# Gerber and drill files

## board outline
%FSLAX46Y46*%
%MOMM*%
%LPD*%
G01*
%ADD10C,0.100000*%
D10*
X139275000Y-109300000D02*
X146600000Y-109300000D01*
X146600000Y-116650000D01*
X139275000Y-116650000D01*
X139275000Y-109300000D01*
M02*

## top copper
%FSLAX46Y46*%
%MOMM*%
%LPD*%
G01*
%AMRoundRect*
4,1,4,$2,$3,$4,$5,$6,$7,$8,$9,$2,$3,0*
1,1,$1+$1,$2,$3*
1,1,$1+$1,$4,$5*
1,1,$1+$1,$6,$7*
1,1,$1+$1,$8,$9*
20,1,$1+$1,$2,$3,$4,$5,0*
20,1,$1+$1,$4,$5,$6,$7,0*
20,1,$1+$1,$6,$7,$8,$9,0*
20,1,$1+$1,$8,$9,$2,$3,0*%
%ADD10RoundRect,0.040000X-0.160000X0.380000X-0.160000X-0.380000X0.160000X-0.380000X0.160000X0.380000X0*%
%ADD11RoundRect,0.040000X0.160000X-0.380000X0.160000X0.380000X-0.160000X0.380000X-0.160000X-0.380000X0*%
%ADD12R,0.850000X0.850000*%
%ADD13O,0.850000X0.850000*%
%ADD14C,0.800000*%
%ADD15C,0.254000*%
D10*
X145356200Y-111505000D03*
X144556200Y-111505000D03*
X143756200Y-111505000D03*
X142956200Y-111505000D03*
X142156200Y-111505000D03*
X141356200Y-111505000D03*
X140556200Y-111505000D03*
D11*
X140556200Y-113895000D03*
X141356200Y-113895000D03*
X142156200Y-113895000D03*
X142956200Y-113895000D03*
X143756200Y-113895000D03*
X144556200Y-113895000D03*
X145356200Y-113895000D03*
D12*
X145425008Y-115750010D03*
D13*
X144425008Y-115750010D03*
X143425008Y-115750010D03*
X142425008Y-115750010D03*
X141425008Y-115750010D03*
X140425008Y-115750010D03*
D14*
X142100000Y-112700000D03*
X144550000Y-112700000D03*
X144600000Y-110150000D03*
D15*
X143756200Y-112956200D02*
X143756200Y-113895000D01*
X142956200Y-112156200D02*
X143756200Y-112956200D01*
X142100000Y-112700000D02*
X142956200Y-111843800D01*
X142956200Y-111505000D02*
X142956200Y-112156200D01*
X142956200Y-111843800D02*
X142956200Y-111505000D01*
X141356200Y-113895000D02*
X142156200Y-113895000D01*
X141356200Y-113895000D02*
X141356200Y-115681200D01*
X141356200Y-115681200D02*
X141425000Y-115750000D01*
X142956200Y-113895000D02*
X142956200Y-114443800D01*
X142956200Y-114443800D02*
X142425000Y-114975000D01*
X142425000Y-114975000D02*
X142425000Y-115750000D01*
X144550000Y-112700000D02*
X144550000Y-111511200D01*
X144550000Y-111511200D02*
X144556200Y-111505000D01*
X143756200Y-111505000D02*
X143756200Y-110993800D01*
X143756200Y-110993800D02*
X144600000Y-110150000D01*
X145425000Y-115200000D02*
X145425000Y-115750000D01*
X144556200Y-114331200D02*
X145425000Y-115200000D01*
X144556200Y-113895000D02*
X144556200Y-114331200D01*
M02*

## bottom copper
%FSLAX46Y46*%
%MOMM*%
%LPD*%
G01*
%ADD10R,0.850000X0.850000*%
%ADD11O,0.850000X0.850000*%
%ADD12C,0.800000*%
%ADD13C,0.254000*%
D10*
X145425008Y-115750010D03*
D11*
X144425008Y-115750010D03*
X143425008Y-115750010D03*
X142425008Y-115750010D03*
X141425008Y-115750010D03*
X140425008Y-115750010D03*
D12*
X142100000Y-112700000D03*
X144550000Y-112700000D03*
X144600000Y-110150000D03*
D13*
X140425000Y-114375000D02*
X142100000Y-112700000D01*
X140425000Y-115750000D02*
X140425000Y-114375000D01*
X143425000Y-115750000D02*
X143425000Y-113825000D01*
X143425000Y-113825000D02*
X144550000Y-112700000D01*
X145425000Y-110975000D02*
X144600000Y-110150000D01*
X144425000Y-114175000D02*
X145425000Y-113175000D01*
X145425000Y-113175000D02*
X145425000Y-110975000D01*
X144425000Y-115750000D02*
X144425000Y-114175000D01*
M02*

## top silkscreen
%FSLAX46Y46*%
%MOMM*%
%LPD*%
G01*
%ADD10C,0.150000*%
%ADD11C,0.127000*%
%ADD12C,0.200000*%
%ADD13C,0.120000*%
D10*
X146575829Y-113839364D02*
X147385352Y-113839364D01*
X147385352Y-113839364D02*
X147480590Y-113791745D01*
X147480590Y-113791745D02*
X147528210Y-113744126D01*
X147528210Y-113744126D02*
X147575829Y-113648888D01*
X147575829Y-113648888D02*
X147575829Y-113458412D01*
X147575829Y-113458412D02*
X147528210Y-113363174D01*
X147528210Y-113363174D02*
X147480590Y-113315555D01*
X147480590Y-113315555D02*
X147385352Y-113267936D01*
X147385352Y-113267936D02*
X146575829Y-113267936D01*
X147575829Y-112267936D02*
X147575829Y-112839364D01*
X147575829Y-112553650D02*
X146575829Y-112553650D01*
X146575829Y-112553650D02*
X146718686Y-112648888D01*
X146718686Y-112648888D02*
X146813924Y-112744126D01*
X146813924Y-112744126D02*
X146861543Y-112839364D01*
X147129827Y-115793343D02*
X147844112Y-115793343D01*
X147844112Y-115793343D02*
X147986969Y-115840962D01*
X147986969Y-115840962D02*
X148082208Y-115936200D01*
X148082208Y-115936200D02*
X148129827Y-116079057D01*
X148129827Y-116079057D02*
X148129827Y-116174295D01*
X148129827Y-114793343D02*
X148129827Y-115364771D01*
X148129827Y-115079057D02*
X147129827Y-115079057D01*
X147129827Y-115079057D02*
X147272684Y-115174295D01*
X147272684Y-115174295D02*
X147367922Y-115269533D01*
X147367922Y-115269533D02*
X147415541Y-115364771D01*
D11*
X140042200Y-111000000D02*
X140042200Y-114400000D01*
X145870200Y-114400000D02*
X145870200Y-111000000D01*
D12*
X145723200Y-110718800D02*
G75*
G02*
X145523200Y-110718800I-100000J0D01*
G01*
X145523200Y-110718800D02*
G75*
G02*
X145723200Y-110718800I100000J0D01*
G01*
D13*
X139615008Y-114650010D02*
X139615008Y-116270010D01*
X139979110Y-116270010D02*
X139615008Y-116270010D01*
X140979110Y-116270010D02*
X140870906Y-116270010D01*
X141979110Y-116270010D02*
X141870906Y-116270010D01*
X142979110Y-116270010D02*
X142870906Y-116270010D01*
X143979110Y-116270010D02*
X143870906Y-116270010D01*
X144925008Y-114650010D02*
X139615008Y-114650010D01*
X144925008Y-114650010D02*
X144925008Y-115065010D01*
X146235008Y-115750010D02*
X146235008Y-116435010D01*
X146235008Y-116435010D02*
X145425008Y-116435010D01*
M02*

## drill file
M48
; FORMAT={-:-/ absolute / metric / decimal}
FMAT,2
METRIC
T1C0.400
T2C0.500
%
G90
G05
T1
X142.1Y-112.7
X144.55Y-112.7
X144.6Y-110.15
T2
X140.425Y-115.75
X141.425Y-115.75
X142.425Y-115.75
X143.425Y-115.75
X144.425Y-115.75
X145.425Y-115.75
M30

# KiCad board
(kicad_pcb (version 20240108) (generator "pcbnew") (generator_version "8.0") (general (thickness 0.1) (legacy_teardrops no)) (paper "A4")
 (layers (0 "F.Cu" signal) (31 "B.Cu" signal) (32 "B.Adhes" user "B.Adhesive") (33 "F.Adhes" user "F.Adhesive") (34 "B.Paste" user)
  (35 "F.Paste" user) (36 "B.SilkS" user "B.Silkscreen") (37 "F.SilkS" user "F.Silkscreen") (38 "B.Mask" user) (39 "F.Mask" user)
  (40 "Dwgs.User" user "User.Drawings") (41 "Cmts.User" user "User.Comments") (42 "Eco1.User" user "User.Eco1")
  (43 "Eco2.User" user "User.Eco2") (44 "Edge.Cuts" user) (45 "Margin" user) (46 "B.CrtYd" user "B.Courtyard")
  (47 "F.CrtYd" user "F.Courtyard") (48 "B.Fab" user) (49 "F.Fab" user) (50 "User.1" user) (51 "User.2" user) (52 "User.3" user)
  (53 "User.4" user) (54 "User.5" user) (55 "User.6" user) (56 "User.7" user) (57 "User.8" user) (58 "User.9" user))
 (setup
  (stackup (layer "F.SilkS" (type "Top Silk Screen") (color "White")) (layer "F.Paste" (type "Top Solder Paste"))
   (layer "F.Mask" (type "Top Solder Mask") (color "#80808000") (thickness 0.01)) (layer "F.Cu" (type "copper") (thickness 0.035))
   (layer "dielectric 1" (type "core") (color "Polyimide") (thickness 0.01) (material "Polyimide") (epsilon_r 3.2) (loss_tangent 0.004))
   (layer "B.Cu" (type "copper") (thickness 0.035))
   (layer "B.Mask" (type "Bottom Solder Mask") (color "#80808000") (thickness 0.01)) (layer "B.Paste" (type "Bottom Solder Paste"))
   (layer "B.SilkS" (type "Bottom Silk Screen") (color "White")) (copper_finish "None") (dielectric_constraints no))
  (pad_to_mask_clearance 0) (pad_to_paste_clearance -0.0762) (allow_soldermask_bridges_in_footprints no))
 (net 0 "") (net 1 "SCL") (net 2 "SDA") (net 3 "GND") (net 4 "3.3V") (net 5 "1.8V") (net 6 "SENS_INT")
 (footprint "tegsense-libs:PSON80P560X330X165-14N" (layer "F.Cu") (at 142.9562 112.7 -90)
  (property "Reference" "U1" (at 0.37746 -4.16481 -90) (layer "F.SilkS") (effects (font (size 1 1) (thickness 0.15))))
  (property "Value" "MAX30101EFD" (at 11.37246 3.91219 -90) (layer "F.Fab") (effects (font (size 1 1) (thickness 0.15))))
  (fp_line (start -1.7 2.914) (end 1.7 2.914) (stroke (width 0.127) (type solid)) (layer "F.SilkS"))
  (fp_line (start 1.7 -2.914) (end -1.7 -2.914) (stroke (width 0.127) (type solid)) (layer "F.SilkS"))
  (fp_circle (center -1.9812 -2.667) (end -1.8812 -2.667) (stroke (width 0.2) (type solid)) (fill none) (layer "F.SilkS"))
  (pad "1" smd roundrect (at -1.195 -2.4 270) (size 0.84 0.4) (layers "F.Cu" "F.Paste" "F.Mask") (roundrect_rratio 0.1))
  (pad "2" smd roundrect (at -1.195 -1.6 270) (size 0.84 0.4) (layers "F.Cu" "F.Paste" "F.Mask") (roundrect_rratio 0.1) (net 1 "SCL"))
  (pad "3" smd roundrect (at -1.195 -0.8 270) (size 0.84 0.4) (layers "F.Cu" "F.Paste" "F.Mask") (roundrect_rratio 0.1) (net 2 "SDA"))
  (pad "4" smd roundrect (at -1.195 0 270) (size 0.84 0.4) (layers "F.Cu" "F.Paste" "F.Mask") (roundrect_rratio 0.1) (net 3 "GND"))
  (pad "5" smd roundrect (at -1.195 0.8 270) (size 0.84 0.4) (layers "F.Cu" "F.Paste" "F.Mask") (roundrect_rratio 0.1))
  (pad "6" smd roundrect (at -1.195 1.6 270) (size 0.84 0.4) (layers "F.Cu" "F.Paste" "F.Mask") (roundrect_rratio 0.1))
  (pad "7" smd roundrect (at -1.195 2.4 270) (size 0.84 0.4) (layers "F.Cu" "F.Paste" "F.Mask") (roundrect_rratio 0.1))
  (pad "8" smd roundrect (at 1.195 2.4 90) (size 0.84 0.4) (layers "F.Cu" "F.Paste" "F.Mask") (roundrect_rratio 0.1))
  (pad "9" smd roundrect (at 1.195 1.6 90) (size 0.84 0.4) (layers "F.Cu" "F.Paste" "F.Mask") (roundrect_rratio 0.1) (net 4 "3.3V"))
  (pad "10" smd roundrect (at 1.195 0.8 90) (size 0.84 0.4) (layers "F.Cu" "F.Paste" "F.Mask") (roundrect_rratio 0.1) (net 4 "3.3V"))
  (pad "11" smd roundrect (at 1.195 0 90) (size 0.84 0.4) (layers "F.Cu" "F.Paste" "F.Mask") (roundrect_rratio 0.1) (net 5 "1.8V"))
  (pad "12" smd roundrect (at 1.195 -0.8 90) (size 0.84 0.4) (layers "F.Cu" "F.Paste" "F.Mask") (roundrect_rratio 0.1) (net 3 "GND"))
  (pad "13" smd roundrect (at 1.195 -1.6 90) (size 0.84 0.4) (layers "F.Cu" "F.Paste" "F.Mask") (roundrect_rratio 0.1) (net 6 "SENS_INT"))
  (pad "14" smd roundrect (at 1.195 -2.4 90) (size 0.84 0.4) (layers "F.Cu" "F.Paste" "F.Mask") (roundrect_rratio 0.1)))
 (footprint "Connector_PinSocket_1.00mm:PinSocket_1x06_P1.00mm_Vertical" (layer "F.Cu") (at 145.425008 115.75001 -90)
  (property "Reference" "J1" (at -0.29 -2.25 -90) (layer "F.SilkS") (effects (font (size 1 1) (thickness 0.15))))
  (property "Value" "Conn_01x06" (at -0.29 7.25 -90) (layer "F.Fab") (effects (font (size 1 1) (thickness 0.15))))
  (fp_line (start -1.1 5.81) (end 0.52 5.81) (stroke (width 0.12) (type solid)) (layer "F.SilkS"))
  (fp_line (start 0.52 5.445898) (end 0.52 5.81) (stroke (width 0.12) (type solid)) (layer "F.SilkS"))
  (fp_line (start 0.52 4.445898) (end 0.52 4.554102) (stroke (width 0.12) (type solid)) (layer "F.SilkS"))
  (fp_line (start 0.52 3.445898) (end 0.52 3.554102) (stroke (width 0.12) (type solid)) (layer "F.SilkS"))
  (fp_line (start 0.52 2.445898) (end 0.52 2.554102) (stroke (width 0.12) (type solid)) (layer "F.SilkS"))
  (fp_line (start 0.52 1.445898) (end 0.52 1.554102) (stroke (width 0.12) (type solid)) (layer "F.SilkS"))
  (fp_line (start -1.1 0.5) (end -1.1 5.81) (stroke (width 0.12) (type solid)) (layer "F.SilkS"))
  (fp_line (start -1.1 0.5) (end -0.685 0.5) (stroke (width 0.12) (type solid)) (layer "F.SilkS"))
  (fp_line (start 0 -0.81) (end 0.685 -0.81) (stroke (width 0.12) (type solid)) (layer "F.SilkS"))
  (fp_line (start 0.685 -0.81) (end 0.685 0) (stroke (width 0.12) (type solid)) (layer "F.SilkS"))
  (pad "1" thru_hole rect (at 0 0 270) (size 0.85 0.85) (drill 0.5) (layers "*.Cu" "*.Mask") (remove_unused_layers no) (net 6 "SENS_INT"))
  (pad "2" thru_hole oval (at 0 1 270) (size 0.85 0.85) (drill 0.5) (layers "*.Cu" "*.Mask") (remove_unused_layers no) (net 2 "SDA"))
  (pad "3" thru_hole oval (at 0 2 270) (size 0.85 0.85) (drill 0.5) (layers "*.Cu" "*.Mask") (remove_unused_layers no) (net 1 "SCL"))
  (pad "4" thru_hole oval (at 0 3 270) (size 0.85 0.85) (drill 0.5) (layers "*.Cu" "*.Mask") (remove_unused_layers no) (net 5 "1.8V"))
  (pad "5" thru_hole oval (at 0 4 270) (size 0.85 0.85) (drill 0.5) (layers "*.Cu" "*.Mask") (remove_unused_layers no) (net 4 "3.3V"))
  (pad "6" thru_hole oval (at 0 5 270) (size 0.85 0.85) (drill 0.5) (layers "*.Cu" "*.Mask") (remove_unused_layers no) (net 3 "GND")))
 (gr_rect (start 139.275 109.3) (end 146.6 116.65) (stroke (width 0.1) (type solid)) (fill none) (layer "Edge.Cuts"))
 (segment (start 143.7562 112.9562) (end 143.7562 113.895) (width 0.254) (layer "F.Cu") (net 3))
 (segment (start 142.9562 112.1562) (end 143.7562 112.9562) (width 0.254) (layer "F.Cu") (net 3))
 (segment (start 142.1 112.7) (end 142.9562 111.8438) (width 0.254) (layer "F.Cu") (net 3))
 (segment (start 142.9562 111.505) (end 142.9562 112.1562) (width 0.254) (layer "F.Cu") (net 3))
 (segment (start 142.9562 111.8438) (end 142.9562 111.505) (width 0.254) (layer "F.Cu") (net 3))
 (via (at 142.1 112.7) (size 0.8) (drill 0.4) (layers "F.Cu" "B.Cu") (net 3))
 (segment (start 140.425 114.375) (end 142.1 112.7) (width 0.254) (layer "B.Cu") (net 3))
 (segment (start 140.425 115.75) (end 140.425 114.375) (width 0.254) (layer "B.Cu") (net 3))
 (segment (start 141.3562 113.895) (end 142.1562 113.895) (width 0.254) (layer "F.Cu") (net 4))
 (segment (start 141.3562 113.895) (end 141.3562 115.6812) (width 0.254) (layer "F.Cu") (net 4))
 (segment (start 141.3562 115.6812) (end 141.425 115.75) (width 0.254) (layer "F.Cu") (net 4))
 (segment (start 142.9562 113.895) (end 142.9562 114.4438) (width 0.254) (layer "F.Cu") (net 5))
 (segment (start 142.9562 114.4438) (end 142.425 114.975) (width 0.254) (layer "F.Cu") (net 5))
 (segment (start 142.425 114.975) (end 142.425 115.75) (width 0.254) (layer "F.Cu") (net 5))
 (segment (start 144.55 112.7) (end 144.55 111.5112) (width 0.254) (layer "F.Cu") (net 1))
 (segment (start 144.55 111.5112) (end 144.5562 111.505) (width 0.254) (layer "F.Cu") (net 1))
 (via (at 144.55 112.7) (size 0.8) (drill 0.4) (layers "F.Cu" "B.Cu") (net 1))
 (segment (start 143.425 115.75) (end 143.425 113.825) (width 0.254) (layer "B.Cu") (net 1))
 (segment (start 143.425 113.825) (end 144.55 112.7) (width 0.254) (layer "B.Cu") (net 1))
 (segment (start 143.7562 111.505) (end 143.7562 110.9938) (width 0.254) (layer "F.Cu") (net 2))
 (segment (start 143.7562 110.9938) (end 144.6 110.15) (width 0.254) (layer "F.Cu") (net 2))
 (via (at 144.6 110.15) (size 0.8) (drill 0.4) (layers "F.Cu" "B.Cu") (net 2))
 (segment (start 145.425 110.975) (end 144.6 110.15) (width 0.254) (layer "B.Cu") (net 2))
 (segment (start 144.425 114.175) (end 145.425 113.175) (width 0.254) (layer "B.Cu") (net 2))
 (segment (start 145.425 113.175) (end 145.425 110.975) (width 0.254) (layer "B.Cu") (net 2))
 (segment (start 144.425 115.75) (end 144.425 114.175) (width 0.254) (layer "B.Cu") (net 2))
 (segment (start 145.425 115.2) (end 145.425 115.75) (width 0.254) (layer "F.Cu") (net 6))
 (segment (start 144.5562 114.3312) (end 145.425 115.2) (width 0.254) (layer "F.Cu") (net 6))
 (segment (start 144.5562 113.895) (end 144.5562 114.3312) (width 0.254) (layer "F.Cu") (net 6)))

